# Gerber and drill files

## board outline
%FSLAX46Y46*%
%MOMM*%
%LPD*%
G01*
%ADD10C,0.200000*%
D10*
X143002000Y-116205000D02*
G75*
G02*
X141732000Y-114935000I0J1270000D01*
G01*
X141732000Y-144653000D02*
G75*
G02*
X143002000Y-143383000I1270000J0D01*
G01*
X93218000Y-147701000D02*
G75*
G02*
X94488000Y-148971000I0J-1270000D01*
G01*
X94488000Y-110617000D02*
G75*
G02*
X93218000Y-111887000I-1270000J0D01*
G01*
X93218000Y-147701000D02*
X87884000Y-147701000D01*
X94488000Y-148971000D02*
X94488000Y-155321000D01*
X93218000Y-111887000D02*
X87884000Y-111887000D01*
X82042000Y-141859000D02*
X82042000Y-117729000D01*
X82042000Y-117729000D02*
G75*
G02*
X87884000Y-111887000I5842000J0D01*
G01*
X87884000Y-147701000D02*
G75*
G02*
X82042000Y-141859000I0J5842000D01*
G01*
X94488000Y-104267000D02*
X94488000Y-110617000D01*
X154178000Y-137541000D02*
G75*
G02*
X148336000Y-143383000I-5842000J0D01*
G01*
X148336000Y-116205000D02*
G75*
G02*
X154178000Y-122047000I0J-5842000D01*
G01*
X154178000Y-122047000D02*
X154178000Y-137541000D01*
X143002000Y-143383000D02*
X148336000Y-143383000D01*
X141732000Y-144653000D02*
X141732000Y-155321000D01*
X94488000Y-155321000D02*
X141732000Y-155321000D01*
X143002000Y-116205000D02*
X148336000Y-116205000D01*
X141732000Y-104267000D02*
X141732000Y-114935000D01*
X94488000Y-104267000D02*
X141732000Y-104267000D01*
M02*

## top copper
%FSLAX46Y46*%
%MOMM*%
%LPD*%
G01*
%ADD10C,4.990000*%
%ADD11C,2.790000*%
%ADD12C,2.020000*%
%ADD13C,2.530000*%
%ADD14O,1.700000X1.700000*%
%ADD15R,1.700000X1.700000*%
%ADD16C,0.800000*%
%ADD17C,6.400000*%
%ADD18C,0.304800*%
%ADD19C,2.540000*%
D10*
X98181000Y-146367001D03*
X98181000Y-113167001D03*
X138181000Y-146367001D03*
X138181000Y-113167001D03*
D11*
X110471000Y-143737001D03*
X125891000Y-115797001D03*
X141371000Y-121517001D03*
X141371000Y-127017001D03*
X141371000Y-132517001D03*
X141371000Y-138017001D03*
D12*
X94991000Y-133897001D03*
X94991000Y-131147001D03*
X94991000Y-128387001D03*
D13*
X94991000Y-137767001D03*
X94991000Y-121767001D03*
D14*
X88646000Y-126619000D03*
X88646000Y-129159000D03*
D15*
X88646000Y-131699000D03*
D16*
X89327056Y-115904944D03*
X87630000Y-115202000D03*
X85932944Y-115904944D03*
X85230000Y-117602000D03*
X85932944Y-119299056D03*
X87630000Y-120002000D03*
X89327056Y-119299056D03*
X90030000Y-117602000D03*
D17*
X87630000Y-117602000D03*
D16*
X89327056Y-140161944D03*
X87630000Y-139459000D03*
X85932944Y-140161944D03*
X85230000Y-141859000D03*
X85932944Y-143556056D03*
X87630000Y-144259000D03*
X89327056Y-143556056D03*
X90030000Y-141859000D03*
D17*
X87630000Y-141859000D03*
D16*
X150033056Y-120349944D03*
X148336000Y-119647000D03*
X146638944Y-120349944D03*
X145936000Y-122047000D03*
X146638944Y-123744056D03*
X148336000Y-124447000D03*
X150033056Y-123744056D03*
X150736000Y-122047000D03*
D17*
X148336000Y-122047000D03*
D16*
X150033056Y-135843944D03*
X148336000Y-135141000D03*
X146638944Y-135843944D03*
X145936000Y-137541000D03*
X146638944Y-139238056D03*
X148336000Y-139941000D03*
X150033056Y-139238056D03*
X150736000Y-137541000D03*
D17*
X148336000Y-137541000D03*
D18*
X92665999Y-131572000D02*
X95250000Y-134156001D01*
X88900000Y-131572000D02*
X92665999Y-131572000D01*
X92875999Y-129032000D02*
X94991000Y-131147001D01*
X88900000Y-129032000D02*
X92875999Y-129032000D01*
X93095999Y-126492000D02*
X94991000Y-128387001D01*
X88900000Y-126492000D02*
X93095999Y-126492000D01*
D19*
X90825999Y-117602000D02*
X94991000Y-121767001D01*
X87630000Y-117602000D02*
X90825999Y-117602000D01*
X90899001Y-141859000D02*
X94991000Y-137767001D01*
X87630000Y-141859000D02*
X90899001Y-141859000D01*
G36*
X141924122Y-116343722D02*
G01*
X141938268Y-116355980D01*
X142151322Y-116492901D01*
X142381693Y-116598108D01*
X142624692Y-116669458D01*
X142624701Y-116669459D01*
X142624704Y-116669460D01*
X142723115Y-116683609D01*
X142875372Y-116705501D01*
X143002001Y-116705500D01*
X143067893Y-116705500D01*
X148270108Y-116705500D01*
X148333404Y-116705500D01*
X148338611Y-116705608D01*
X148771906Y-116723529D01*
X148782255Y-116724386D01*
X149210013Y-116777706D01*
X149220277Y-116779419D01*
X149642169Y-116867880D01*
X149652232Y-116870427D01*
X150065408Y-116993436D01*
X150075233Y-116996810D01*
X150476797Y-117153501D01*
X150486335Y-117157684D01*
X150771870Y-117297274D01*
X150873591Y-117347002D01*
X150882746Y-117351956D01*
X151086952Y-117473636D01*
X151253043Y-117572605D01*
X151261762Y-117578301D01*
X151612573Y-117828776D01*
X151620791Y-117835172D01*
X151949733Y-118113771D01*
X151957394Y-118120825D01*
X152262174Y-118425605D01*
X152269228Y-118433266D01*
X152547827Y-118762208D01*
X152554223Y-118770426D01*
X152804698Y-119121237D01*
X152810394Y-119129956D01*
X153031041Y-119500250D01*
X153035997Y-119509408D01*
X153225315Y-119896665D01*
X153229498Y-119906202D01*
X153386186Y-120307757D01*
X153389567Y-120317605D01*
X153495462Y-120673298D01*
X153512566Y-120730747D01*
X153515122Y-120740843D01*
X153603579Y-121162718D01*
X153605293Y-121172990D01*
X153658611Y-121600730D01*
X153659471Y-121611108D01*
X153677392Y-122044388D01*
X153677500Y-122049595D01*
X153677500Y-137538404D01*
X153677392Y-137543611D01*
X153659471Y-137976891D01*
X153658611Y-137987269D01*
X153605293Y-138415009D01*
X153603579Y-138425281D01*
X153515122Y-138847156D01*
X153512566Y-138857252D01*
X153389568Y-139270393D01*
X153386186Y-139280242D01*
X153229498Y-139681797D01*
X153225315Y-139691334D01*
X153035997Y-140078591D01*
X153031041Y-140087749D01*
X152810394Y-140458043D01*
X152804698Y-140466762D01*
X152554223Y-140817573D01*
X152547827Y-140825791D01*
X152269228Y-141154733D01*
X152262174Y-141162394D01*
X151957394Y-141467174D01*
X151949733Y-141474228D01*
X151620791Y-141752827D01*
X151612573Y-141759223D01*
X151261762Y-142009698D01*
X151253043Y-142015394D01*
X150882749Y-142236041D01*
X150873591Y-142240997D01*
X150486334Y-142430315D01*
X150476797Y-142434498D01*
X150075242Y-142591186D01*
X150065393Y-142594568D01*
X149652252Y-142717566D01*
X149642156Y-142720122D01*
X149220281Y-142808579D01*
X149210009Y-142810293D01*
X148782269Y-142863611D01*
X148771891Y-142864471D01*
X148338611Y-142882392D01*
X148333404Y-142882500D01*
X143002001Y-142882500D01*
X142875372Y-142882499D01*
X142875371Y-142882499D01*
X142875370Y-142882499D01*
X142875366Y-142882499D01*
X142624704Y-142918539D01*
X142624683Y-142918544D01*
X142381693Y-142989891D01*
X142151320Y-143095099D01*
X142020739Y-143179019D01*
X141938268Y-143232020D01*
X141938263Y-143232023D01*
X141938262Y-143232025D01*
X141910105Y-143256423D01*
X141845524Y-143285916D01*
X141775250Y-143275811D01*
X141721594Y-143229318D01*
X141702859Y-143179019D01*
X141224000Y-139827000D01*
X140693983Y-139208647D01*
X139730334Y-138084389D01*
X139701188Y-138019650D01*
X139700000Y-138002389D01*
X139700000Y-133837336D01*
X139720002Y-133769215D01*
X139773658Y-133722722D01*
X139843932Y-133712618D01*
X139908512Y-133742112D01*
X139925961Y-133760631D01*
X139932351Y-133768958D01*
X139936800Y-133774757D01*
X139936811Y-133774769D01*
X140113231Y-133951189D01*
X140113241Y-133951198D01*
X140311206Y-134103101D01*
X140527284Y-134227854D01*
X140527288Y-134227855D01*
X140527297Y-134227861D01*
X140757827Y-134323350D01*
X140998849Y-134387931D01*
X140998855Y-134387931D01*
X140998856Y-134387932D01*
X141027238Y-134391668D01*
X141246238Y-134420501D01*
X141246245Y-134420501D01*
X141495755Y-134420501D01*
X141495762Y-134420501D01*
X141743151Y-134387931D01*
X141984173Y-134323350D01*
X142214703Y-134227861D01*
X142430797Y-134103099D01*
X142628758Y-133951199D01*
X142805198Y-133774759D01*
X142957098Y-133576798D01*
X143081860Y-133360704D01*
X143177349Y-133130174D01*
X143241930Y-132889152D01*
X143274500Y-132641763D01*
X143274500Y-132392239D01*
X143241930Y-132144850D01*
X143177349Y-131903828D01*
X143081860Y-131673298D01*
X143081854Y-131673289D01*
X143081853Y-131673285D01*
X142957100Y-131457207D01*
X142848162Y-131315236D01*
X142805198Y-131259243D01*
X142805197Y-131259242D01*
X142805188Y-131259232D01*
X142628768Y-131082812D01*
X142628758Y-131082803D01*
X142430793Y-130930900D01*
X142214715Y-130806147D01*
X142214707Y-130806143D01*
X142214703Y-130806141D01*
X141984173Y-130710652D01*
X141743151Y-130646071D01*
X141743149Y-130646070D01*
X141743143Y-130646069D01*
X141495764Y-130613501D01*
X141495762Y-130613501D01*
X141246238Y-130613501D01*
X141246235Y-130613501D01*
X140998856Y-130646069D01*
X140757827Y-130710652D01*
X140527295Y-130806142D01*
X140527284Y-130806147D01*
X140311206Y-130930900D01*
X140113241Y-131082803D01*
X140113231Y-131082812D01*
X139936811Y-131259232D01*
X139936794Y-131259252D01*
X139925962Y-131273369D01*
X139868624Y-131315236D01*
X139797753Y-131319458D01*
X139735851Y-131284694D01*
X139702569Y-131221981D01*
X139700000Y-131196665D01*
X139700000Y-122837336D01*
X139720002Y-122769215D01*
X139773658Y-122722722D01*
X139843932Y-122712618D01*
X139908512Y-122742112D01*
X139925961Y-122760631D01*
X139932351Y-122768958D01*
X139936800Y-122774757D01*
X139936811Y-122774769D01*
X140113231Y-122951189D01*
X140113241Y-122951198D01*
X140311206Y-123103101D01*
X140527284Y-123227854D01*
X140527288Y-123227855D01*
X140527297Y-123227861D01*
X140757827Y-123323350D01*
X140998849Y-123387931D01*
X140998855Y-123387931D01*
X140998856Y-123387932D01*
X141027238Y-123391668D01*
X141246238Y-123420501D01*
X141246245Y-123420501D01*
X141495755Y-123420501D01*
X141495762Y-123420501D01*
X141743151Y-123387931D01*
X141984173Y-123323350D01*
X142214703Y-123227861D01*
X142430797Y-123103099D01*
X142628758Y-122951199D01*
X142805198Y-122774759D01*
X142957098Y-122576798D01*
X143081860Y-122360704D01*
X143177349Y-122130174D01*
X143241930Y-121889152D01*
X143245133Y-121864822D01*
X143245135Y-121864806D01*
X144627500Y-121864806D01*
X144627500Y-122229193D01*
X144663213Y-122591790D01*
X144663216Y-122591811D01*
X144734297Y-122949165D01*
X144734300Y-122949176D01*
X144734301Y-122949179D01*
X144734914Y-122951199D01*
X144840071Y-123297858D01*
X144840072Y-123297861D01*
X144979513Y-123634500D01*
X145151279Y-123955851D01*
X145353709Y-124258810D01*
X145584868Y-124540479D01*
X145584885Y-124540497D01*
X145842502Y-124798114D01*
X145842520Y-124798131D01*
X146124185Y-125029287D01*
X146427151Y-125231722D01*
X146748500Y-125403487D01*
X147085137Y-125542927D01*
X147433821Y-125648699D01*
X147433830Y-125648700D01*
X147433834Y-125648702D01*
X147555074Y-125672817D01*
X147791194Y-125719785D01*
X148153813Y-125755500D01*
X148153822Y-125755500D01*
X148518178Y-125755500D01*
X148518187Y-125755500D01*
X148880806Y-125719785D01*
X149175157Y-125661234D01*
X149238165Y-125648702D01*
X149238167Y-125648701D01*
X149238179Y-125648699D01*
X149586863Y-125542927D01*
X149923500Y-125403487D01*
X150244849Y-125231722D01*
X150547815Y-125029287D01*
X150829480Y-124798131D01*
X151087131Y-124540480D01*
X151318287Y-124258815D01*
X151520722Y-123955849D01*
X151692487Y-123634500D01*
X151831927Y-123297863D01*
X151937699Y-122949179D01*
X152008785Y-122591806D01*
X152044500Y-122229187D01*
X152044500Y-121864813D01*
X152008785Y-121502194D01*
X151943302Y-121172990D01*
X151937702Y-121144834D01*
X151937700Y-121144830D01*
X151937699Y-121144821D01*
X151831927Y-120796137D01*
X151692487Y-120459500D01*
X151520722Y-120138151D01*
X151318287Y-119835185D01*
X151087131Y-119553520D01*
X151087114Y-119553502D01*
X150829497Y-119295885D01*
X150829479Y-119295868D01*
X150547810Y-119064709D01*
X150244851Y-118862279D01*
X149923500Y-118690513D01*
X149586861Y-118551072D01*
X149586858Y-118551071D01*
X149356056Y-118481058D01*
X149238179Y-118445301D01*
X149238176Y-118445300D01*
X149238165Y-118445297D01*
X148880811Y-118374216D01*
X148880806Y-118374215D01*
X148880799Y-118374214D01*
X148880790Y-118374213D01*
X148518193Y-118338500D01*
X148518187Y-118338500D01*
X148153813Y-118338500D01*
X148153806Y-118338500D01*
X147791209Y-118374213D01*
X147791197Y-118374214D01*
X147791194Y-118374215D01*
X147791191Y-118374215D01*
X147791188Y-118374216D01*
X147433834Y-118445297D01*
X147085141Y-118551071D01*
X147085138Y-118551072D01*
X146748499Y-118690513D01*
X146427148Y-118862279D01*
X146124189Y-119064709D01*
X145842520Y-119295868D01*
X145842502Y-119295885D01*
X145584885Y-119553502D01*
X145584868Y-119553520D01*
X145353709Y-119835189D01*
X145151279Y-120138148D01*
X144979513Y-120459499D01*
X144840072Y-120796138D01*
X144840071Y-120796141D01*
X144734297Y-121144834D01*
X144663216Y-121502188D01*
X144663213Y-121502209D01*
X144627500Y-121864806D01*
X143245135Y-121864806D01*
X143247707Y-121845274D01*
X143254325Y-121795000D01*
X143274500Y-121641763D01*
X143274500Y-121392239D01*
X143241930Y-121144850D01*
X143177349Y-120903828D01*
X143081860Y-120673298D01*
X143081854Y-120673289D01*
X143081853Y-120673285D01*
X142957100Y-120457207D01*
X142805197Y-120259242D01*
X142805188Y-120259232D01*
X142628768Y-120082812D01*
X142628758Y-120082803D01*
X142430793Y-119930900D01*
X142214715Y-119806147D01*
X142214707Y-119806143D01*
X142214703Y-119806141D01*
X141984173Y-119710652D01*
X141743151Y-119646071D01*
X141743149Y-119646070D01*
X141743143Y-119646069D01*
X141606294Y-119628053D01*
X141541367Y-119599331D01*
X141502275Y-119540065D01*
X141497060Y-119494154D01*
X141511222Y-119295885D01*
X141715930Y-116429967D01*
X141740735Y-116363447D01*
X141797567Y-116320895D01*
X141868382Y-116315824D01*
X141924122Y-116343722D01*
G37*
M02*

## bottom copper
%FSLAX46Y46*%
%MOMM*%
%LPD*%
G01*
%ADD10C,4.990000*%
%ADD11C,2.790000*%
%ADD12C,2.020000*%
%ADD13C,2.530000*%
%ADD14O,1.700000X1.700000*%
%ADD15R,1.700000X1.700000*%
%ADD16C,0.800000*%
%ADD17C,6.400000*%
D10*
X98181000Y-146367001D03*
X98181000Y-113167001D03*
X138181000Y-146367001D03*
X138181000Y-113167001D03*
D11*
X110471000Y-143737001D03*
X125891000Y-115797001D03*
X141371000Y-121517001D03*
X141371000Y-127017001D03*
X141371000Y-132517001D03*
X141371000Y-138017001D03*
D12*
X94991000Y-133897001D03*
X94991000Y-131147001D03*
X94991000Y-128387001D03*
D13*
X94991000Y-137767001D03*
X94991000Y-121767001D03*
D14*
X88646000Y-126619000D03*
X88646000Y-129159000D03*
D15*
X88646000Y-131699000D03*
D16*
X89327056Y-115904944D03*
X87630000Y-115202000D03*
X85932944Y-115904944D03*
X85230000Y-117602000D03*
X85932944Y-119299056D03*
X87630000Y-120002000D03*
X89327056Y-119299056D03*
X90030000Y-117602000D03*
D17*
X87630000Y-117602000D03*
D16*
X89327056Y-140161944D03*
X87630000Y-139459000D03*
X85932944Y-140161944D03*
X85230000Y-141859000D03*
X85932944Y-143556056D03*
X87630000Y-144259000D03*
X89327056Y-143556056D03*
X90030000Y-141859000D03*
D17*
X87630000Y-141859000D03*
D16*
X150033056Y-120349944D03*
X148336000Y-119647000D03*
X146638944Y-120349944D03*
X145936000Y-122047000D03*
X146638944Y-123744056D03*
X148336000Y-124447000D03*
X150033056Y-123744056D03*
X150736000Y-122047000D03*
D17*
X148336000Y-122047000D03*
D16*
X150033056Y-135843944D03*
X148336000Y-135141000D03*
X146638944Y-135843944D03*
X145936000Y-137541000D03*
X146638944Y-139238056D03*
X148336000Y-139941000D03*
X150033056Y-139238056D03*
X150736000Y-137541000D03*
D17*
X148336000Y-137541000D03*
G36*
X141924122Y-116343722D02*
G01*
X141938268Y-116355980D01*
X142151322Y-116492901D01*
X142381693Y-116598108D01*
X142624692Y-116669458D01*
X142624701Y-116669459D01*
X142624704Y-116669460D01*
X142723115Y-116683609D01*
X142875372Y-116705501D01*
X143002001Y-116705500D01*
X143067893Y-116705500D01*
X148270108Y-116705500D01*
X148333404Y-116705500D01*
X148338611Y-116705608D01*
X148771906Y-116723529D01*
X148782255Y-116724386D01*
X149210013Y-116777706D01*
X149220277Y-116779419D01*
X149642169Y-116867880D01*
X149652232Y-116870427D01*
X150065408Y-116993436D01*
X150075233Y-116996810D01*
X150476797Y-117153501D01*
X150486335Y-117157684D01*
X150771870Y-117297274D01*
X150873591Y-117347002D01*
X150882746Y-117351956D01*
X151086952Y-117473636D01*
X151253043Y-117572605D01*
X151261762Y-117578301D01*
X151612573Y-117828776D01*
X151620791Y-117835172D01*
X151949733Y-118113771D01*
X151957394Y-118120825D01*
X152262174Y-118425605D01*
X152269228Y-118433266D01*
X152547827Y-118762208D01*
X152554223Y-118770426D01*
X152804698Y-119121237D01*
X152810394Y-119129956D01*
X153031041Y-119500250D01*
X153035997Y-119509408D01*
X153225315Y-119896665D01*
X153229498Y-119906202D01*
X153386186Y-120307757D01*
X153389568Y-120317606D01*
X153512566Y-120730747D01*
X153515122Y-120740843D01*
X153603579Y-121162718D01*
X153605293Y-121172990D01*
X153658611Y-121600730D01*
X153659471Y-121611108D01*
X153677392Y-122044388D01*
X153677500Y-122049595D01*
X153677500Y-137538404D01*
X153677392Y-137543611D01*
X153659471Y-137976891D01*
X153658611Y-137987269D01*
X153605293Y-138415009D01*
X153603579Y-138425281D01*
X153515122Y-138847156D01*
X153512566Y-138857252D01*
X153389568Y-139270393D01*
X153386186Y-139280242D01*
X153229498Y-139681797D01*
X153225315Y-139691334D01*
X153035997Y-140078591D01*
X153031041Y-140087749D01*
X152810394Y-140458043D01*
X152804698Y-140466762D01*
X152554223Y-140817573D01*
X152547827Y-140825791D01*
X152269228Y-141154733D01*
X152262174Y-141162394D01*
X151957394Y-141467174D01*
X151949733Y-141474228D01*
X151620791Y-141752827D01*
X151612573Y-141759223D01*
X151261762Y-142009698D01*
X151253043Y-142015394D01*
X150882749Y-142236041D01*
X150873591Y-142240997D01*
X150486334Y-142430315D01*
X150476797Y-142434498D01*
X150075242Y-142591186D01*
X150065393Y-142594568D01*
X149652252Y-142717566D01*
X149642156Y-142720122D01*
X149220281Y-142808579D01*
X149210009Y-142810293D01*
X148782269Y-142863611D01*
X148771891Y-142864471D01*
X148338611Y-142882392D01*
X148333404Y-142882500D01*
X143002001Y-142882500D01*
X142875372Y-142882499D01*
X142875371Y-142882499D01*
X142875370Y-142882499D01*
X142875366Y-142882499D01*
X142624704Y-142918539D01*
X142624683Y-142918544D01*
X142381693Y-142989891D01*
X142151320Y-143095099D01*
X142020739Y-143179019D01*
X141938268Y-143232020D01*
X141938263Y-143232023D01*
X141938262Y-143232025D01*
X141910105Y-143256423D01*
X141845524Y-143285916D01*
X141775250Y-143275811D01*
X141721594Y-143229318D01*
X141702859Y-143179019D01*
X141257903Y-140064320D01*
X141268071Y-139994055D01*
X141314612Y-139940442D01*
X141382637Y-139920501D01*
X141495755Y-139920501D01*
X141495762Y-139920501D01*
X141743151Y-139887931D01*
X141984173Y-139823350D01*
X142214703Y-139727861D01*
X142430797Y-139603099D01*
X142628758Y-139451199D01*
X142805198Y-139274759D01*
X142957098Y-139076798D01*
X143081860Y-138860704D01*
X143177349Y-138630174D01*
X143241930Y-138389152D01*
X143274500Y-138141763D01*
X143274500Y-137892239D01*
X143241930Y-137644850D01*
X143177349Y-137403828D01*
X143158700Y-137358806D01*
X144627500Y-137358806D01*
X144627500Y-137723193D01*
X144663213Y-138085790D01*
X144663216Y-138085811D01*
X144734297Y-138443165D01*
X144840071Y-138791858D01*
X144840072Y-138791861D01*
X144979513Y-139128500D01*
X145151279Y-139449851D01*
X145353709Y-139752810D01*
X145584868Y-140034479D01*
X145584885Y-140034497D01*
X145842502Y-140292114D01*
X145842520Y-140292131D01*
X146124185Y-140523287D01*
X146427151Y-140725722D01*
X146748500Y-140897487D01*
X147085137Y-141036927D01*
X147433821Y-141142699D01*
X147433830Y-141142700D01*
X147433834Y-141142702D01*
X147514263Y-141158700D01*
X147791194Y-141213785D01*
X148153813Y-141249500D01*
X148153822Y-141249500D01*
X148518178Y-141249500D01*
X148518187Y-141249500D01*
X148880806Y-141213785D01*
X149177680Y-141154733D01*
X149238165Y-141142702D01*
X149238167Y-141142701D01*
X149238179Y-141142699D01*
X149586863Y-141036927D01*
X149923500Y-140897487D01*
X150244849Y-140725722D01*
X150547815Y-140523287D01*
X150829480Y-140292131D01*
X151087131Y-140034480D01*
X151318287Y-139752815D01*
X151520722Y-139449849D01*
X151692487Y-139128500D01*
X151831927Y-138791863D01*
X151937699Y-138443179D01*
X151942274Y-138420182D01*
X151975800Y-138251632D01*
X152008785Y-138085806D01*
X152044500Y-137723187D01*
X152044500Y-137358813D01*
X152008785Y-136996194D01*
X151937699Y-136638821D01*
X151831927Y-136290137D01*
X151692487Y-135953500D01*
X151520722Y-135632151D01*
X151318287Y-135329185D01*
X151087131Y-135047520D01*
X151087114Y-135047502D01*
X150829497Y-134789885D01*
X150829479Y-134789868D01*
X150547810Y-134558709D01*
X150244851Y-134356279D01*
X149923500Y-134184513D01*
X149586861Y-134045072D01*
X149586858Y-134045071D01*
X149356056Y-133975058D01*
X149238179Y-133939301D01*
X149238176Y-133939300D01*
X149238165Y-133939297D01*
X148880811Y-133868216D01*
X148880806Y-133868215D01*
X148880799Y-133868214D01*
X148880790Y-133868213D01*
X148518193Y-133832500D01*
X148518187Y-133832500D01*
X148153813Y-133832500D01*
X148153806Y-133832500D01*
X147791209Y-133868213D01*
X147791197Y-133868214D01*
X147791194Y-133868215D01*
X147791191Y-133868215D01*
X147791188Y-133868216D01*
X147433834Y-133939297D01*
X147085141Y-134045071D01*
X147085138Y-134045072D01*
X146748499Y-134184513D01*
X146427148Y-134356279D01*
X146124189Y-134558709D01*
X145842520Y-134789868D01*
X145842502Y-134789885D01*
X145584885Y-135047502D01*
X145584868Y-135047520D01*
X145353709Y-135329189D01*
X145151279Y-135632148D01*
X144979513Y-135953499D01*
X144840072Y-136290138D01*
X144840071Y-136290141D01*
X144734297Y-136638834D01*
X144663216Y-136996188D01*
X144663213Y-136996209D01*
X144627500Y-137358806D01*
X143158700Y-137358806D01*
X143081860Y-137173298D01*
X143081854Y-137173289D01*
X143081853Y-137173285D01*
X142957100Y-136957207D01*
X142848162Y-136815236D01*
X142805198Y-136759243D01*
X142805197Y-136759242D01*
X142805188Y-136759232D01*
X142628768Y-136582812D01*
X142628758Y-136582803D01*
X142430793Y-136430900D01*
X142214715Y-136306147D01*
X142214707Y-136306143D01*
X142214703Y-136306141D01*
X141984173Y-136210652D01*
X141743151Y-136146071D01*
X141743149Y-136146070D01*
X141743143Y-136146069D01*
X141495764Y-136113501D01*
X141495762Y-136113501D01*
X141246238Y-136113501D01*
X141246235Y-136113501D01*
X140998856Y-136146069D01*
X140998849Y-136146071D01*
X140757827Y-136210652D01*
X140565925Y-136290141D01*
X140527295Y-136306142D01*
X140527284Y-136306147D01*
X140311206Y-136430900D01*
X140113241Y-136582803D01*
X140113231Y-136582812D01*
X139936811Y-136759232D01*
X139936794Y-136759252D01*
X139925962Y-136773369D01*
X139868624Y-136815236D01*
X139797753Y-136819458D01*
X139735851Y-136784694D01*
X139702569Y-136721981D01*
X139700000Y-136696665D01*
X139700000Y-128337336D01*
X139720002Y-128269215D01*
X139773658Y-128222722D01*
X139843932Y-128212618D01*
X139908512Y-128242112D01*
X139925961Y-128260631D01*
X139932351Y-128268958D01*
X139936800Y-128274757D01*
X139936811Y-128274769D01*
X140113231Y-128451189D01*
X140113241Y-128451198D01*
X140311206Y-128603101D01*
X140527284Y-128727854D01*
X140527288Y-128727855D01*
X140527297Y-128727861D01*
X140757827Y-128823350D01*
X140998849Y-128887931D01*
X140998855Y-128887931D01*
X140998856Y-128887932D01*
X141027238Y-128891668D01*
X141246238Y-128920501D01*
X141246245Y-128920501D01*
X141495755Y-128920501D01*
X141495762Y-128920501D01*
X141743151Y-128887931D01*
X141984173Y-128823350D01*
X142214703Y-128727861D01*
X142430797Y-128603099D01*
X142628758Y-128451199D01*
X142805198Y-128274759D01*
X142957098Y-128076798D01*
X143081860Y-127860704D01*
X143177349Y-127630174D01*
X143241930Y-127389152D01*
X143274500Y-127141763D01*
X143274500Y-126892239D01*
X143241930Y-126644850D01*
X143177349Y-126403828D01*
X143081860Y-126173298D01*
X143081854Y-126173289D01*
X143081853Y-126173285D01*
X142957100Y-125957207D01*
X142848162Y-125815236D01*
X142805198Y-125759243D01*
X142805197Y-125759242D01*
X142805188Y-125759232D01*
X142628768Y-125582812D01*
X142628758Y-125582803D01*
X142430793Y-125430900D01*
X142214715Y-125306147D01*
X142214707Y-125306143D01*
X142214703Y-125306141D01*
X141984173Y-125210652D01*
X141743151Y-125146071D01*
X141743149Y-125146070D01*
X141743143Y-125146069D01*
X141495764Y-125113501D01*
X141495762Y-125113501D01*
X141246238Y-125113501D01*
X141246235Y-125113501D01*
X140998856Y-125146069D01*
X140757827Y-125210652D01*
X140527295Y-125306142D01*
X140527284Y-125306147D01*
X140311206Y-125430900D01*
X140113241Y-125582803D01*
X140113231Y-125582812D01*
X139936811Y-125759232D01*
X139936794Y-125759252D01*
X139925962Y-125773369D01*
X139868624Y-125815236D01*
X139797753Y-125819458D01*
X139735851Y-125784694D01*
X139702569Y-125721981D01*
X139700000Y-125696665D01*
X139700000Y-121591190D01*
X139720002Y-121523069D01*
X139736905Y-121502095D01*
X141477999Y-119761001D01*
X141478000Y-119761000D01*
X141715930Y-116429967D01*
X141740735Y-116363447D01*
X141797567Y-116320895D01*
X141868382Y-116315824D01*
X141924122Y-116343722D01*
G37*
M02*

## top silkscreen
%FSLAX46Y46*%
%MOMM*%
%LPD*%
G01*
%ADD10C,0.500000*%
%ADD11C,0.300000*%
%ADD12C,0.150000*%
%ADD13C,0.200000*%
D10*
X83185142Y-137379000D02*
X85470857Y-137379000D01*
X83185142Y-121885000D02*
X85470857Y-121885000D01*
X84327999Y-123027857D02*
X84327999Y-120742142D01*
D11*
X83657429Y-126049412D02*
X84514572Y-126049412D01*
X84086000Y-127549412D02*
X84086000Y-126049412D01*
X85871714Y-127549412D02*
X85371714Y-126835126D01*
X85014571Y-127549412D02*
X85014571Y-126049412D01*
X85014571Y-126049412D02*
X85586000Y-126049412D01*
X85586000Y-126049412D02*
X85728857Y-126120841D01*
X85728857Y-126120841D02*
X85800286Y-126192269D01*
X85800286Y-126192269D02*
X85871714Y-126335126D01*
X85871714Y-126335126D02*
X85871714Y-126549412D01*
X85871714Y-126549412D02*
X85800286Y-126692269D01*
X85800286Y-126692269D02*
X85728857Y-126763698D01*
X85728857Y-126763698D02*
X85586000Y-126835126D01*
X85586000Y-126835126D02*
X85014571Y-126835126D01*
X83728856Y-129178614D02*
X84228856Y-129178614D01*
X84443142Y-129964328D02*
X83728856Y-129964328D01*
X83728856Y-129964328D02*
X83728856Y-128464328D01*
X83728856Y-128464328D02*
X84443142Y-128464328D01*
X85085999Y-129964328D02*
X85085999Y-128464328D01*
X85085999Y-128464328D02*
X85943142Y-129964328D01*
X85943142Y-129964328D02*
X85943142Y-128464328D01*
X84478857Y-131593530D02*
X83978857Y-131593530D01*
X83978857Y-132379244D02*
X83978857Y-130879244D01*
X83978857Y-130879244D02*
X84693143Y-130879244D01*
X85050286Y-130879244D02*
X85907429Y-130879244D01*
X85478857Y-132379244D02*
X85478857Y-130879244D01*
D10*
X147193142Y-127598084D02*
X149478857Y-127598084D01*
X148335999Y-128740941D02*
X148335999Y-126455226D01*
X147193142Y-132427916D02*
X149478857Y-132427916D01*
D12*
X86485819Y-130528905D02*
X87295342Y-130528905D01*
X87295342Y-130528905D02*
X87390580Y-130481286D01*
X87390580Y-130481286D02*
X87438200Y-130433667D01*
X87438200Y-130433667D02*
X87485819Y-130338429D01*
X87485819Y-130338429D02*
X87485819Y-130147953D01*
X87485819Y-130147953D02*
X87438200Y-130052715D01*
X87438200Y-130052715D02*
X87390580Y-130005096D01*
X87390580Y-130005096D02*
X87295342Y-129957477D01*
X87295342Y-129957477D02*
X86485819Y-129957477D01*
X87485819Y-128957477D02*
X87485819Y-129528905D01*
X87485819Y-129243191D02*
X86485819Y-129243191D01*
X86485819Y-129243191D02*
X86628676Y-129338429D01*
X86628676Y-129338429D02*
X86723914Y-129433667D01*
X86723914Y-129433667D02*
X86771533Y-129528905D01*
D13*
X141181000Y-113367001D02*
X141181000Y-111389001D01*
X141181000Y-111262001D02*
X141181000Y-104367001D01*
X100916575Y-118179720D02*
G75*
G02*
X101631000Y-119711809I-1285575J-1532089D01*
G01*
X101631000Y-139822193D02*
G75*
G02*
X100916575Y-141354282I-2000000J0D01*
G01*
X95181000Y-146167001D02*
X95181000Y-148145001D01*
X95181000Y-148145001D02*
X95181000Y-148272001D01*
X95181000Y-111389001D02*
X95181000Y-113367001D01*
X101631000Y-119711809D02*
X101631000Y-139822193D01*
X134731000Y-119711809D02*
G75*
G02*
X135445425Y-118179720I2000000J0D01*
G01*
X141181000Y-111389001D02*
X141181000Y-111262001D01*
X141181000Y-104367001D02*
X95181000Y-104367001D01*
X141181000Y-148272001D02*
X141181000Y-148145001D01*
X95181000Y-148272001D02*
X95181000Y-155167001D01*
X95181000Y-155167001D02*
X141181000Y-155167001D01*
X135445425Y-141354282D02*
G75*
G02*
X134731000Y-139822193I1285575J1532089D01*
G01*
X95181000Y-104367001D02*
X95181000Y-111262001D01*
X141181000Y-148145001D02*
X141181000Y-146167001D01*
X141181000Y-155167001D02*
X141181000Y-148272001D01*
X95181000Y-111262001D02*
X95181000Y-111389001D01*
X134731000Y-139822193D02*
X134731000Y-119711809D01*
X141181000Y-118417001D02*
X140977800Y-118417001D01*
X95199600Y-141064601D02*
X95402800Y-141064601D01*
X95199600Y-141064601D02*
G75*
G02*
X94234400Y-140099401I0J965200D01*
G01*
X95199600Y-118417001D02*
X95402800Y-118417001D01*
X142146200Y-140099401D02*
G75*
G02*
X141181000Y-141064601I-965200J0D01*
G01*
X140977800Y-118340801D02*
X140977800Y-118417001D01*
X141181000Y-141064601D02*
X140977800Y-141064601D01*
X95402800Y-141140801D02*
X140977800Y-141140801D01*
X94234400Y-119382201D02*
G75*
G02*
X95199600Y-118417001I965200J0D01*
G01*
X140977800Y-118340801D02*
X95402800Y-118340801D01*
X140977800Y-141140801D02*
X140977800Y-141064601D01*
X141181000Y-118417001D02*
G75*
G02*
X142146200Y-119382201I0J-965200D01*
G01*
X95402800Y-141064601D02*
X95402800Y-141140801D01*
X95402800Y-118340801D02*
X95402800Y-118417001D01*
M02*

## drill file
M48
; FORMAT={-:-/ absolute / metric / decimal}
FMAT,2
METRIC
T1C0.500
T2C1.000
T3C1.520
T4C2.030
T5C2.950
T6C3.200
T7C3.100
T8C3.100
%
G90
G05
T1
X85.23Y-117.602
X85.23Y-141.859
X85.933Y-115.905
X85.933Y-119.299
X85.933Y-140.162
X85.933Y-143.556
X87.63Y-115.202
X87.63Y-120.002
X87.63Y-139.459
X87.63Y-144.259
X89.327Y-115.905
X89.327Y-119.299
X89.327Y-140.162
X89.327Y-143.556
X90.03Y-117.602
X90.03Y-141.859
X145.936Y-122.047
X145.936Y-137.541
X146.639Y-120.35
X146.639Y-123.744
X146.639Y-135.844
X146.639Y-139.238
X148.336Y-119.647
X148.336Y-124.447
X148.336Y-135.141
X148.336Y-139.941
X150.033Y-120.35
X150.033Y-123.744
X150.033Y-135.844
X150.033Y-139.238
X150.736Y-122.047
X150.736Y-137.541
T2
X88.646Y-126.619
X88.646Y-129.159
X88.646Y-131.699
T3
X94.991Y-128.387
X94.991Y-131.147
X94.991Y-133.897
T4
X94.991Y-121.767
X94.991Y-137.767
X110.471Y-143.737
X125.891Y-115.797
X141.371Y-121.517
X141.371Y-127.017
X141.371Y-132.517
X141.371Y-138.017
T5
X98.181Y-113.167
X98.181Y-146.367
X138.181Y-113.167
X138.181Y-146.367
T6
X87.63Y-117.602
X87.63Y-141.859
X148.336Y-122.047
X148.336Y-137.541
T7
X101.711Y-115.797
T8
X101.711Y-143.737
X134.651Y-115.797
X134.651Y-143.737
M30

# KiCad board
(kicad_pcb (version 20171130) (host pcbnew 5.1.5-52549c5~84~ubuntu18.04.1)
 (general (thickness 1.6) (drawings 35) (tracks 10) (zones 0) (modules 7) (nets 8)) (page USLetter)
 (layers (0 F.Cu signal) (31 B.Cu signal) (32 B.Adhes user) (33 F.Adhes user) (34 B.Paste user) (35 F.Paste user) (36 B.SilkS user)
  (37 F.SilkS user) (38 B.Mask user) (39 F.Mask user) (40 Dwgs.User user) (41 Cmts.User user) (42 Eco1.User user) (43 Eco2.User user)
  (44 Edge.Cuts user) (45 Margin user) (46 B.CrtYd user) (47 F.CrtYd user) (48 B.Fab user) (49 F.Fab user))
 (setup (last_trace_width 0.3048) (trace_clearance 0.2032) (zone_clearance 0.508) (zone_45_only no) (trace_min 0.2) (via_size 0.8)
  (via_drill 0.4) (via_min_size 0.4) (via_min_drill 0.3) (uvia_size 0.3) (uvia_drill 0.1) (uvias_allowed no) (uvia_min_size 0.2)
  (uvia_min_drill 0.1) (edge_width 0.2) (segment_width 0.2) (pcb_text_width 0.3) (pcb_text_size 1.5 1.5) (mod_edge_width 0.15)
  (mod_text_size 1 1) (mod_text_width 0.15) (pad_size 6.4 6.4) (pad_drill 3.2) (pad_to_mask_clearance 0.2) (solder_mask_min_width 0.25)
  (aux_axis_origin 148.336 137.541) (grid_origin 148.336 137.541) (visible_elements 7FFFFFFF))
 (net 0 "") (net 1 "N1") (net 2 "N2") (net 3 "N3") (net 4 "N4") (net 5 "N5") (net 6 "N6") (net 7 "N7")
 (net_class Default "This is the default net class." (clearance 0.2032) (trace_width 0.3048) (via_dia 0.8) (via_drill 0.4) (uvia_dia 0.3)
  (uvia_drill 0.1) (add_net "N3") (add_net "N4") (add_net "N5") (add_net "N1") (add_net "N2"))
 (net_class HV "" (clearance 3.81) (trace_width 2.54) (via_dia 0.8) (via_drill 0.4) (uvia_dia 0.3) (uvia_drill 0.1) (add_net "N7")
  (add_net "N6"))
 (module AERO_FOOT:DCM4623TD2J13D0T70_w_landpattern (layer F.Cu) (at 118.181 129.767001)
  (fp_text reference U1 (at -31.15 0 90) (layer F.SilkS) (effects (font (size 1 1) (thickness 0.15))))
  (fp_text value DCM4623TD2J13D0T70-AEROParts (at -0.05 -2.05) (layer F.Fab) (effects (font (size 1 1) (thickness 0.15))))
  (fp_line (start 23 -16.4) (end 23 -18.378) (layer F.SilkS) (width 0.2))
  (fp_line (start 23 -18.505) (end 23 -25.4) (layer F.SilkS) (width 0.2))
  (fp_arc (start -18.55 -10.055192) (end -16.55 -10.055192) (angle -50) (layer F.SilkS) (width 0.2))
  (fp_arc (start -18.55 10.055192) (end -17.264425 11.587281) (angle -50) (layer F.SilkS) (width 0.2))
  (fp_line (start -23 16.4) (end -23 18.378) (layer F.SilkS) (width 0.2))
  (fp_line (start -23 18.378) (end -23 18.505) (layer F.SilkS) (width 0.2))
  (fp_line (start -23 -18.378) (end -23 -16.4) (layer F.SilkS) (width 0.2))
  (fp_line (start -16.55 -10.055192) (end -16.55 10.055192) (layer F.SilkS) (width 0.2))
  (fp_arc (start 18.55 -10.055192) (end 17.264425 -11.587281) (angle -50) (layer F.SilkS) (width 0.2))
  (fp_line (start 23 -18.378) (end 23 -18.505) (layer F.SilkS) (width 0.2))
  (fp_line (start 23 -25.4) (end -23 -25.4) (layer F.SilkS) (width 0.2))
  (fp_line (start 23 18.505) (end 23 18.378) (layer F.SilkS) (width 0.2))
  (fp_line (start -23 18.505) (end -23 25.4) (layer F.SilkS) (width 0.2))
  (fp_line (start -23 25.4) (end 23 25.4) (layer F.SilkS) (width 0.2))
  (fp_arc (start 18.55 10.055192) (end 16.55 10.055192) (angle -50) (layer F.SilkS) (width 0.2))
  (fp_line (start -23 -25.4) (end -23 -18.505) (layer F.SilkS) (width 0.2))
  (fp_line (start 23 18.378) (end 23 16.4) (layer F.SilkS) (width 0.2))
  (fp_line (start 23 25.4) (end 23 18.505) (layer F.SilkS) (width 0.2))
  (fp_line (start -23 -18.505) (end -23 -18.378) (layer F.SilkS) (width 0.2))
  (fp_line (start 16.55 10.055192) (end 16.55 -10.055192) (layer F.SilkS) (width 0.2))
  (fp_line (start 23 -11.35) (end 22.7968 -11.35) (layer F.SilkS) (width 0.2))
  (fp_line (start -22.9814 11.2976) (end -22.7782 11.2976) (layer F.SilkS) (width 0.2))
  (fp_arc (start -22.9814 10.3324) (end -23.9466 10.3324) (angle -90) (layer F.SilkS) (width 0.2))
  (fp_line (start -22.9814 -11.35) (end -22.7782 -11.35) (layer F.SilkS) (width 0.2))
  (fp_arc (start 23 10.3324) (end 23 11.2976) (angle -90) (layer F.SilkS) (width 0.2))
  (fp_line (start 22.7968 -11.4262) (end 22.7968 -11.35) (layer F.SilkS) (width 0.2))
  (fp_line (start 23 11.2976) (end 22.7968 11.2976) (layer F.SilkS) (width 0.2))
  (fp_line (start -22.7782 11.3738) (end 22.7968 11.3738) (layer F.SilkS) (width 0.2))
  (fp_arc (start -22.9814 -10.3848) (end -22.9814 -11.35) (angle -90) (layer F.SilkS) (width 0.2))
  (fp_line (start 22.7968 -11.4262) (end -22.7782 -11.4262) (layer F.SilkS) (width 0.2))
  (fp_line (start 22.7968 11.3738) (end 22.7968 11.2976) (layer F.SilkS) (width 0.2))
  (fp_arc (start 23 -10.3848) (end 23.9652 -10.3848) (angle -90) (layer F.SilkS) (width 0.2))
  (fp_line (start -22.7782 11.2976) (end -22.7782 11.3738) (layer F.SilkS) (width 0.2))
  (fp_line (start -22.7782 -11.4262) (end -22.7782 -11.35) (layer F.SilkS) (width 0.2))
  (pad 14 thru_hole circle (at -20 16.6) (size 4.99 4.99) (drill 2.949999) (layers *.Cu *.Mask))
  (pad 12 thru_hole circle (at -20 -16.6) (size 4.99 4.99) (drill 2.949999) (layers *.Cu *.Mask))
  (pad 15 thru_hole circle (at 20 16.6) (size 4.99 4.99) (drill 2.949999) (layers *.Cu *.Mask))
  (pad 13 thru_hole circle (at 20 -16.6) (size 4.99 4.99) (drill 2.949999) (layers *.Cu *.Mask))
  (pad 10 thru_hole circle (at -7.71 13.97) (size 2.79 2.79) (drill 2.03) (layers *.Cu *.Mask))
  (pad 11 thru_hole circle (at 7.71 -13.97) (size 2.79 2.79) (drill 2.03) (layers *.Cu *.Mask))
  (pad "" np_thru_hole circle (at 16.47 13.97) (size 3.1 3.1) (drill 3.1) (layers *.Cu *.Mask))
  (pad "" np_thru_hole circle (at -16.47 13.97) (size 3.1 3.1) (drill 3.1) (layers *.Cu *.Mask))
  (pad "" np_thru_hole circle (at -16.47 -13.97) (size 3.099999 3.099999) (drill 3.099999) (layers *.Cu *.Mask))
  (pad "" np_thru_hole circle (at 16.47 -13.97) (size 3.1 3.1) (drill 3.1) (layers *.Cu *.Mask))
  (pad 9 thru_hole circle (at 23.19 -8.25) (size 2.79 2.79) (drill 2.03) (layers *.Cu *.Mask) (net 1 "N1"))
  (pad 8 thru_hole circle (at 23.19 -2.75) (size 2.79 2.79) (drill 2.03) (layers *.Cu *.Mask) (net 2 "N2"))
  (pad 7 thru_hole circle (at 23.19 2.75) (size 2.79 2.79) (drill 2.03) (layers *.Cu *.Mask) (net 1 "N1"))
  (pad 6 thru_hole circle (at 23.19 8.25) (size 2.79 2.79) (drill 2.03) (layers *.Cu *.Mask) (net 2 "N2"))
  (pad 4 thru_hole circle (at -23.19 4.13) (size 2.02 2.02) (drill 1.52) (layers *.Cu *.Mask) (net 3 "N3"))
  (pad 3 thru_hole circle (at -23.19 1.38) (size 2.02 2.02) (drill 1.52) (layers *.Cu *.Mask) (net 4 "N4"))
  (pad 2 thru_hole circle (at -23.19 -1.38) (size 2.02 2.02) (drill 1.52) (layers *.Cu *.Mask) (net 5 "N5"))
  (pad 5 thru_hole circle (at -23.19 8) (size 2.53 2.53) (drill 2.03) (layers *.Cu *.Mask) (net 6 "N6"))
  (pad 1 thru_hole circle (at -23.19 -8) (size 2.53 2.53) (drill 2.03) (layers *.Cu *.Mask) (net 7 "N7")))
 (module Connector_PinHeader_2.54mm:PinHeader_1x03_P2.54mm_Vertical (layer B.Cu) (at 88.646 131.699)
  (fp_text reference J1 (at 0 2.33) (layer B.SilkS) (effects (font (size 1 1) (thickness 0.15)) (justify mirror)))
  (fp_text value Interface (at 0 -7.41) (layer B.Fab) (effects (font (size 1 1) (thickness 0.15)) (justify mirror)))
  (pad 3 thru_hole oval (at 0 -5.08) (size 1.7 1.7) (drill 1) (layers *.Cu *.Mask) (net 5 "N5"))
  (pad 2 thru_hole oval (at 0 -2.54) (size 1.7 1.7) (drill 1) (layers *.Cu *.Mask) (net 4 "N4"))
  (pad 1 thru_hole rect (at 0 0) (size 1.7 1.7) (drill 1) (layers *.Cu *.Mask) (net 3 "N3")))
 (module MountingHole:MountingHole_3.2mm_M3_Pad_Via (layer F.Cu) (at 87.63 117.602)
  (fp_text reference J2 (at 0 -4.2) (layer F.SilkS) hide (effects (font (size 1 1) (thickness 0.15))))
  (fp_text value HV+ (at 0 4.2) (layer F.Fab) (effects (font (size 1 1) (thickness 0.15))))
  (pad 1 thru_hole circle (at 1.697056 -1.697056) (size 0.8 0.8) (drill 0.5) (layers *.Cu *.Mask) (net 7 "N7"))
  (pad 1 thru_hole circle (at 0 -2.4) (size 0.8 0.8) (drill 0.5) (layers *.Cu *.Mask) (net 7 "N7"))
  (pad 1 thru_hole circle (at -1.697056 -1.697056) (size 0.8 0.8) (drill 0.5) (layers *.Cu *.Mask) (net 7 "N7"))
  (pad 1 thru_hole circle (at -2.4 0) (size 0.8 0.8) (drill 0.5) (layers *.Cu *.Mask) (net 7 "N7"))
  (pad 1 thru_hole circle (at -1.697056 1.697056) (size 0.8 0.8) (drill 0.5) (layers *.Cu *.Mask) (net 7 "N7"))
  (pad 1 thru_hole circle (at 0 2.4) (size 0.8 0.8) (drill 0.5) (layers *.Cu *.Mask) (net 7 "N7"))
  (pad 1 thru_hole circle (at 1.697056 1.697056) (size 0.8 0.8) (drill 0.5) (layers *.Cu *.Mask) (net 7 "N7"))
  (pad 1 thru_hole circle (at 2.4 0) (size 0.8 0.8) (drill 0.5) (layers *.Cu *.Mask) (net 7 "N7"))
  (pad 1 thru_hole circle (at 0 0) (size 6.4 6.4) (drill 3.2) (layers *.Cu *.Mask) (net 7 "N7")))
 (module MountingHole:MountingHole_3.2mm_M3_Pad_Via (layer F.Cu) (at 87.63 141.859)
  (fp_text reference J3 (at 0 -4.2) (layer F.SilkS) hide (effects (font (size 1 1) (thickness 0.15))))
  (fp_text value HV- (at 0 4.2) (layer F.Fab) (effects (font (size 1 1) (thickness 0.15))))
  (pad 1 thru_hole circle (at 1.697056 -1.697056) (size 0.8 0.8) (drill 0.5) (layers *.Cu *.Mask) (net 6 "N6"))
  (pad 1 thru_hole circle (at 0 -2.4) (size 0.8 0.8) (drill 0.5) (layers *.Cu *.Mask) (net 6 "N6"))
  (pad 1 thru_hole circle (at -1.697056 -1.697056) (size 0.8 0.8) (drill 0.5) (layers *.Cu *.Mask) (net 6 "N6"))
  (pad 1 thru_hole circle (at -2.4 0) (size 0.8 0.8) (drill 0.5) (layers *.Cu *.Mask) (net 6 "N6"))
  (pad 1 thru_hole circle (at -1.697056 1.697056) (size 0.8 0.8) (drill 0.5) (layers *.Cu *.Mask) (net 6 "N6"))
  (pad 1 thru_hole circle (at 0 2.4) (size 0.8 0.8) (drill 0.5) (layers *.Cu *.Mask) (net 6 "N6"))
  (pad 1 thru_hole circle (at 1.697056 1.697056) (size 0.8 0.8) (drill 0.5) (layers *.Cu *.Mask) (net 6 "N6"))
  (pad 1 thru_hole circle (at 2.4 0) (size 0.8 0.8) (drill 0.5) (layers *.Cu *.Mask) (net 6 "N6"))
  (pad 1 thru_hole circle (at 0 0) (size 6.4 6.4) (drill 3.2) (layers *.Cu *.Mask) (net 6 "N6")))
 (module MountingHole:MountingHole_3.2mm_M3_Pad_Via (layer F.Cu) (at 148.336 122.047)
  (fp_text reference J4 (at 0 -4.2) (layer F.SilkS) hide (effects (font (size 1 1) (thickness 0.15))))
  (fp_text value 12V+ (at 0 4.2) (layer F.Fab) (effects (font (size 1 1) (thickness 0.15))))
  (pad 1 thru_hole circle (at 1.697056 -1.697056) (size 0.8 0.8) (drill 0.5) (layers *.Cu *.Mask) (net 1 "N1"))
  (pad 1 thru_hole circle (at 0 -2.4) (size 0.8 0.8) (drill 0.5) (layers *.Cu *.Mask) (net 1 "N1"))
  (pad 1 thru_hole circle (at -1.697056 -1.697056) (size 0.8 0.8) (drill 0.5) (layers *.Cu *.Mask) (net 1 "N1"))
  (pad 1 thru_hole circle (at -2.4 0) (size 0.8 0.8) (drill 0.5) (layers *.Cu *.Mask) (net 1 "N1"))
  (pad 1 thru_hole circle (at -1.697056 1.697056) (size 0.8 0.8) (drill 0.5) (layers *.Cu *.Mask) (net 1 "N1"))
  (pad 1 thru_hole circle (at 0 2.4) (size 0.8 0.8) (drill 0.5) (layers *.Cu *.Mask) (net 1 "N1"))
  (pad 1 thru_hole circle (at 1.697056 1.697056) (size 0.8 0.8) (drill 0.5) (layers *.Cu *.Mask) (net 1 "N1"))
  (pad 1 thru_hole circle (at 2.4 0) (size 0.8 0.8) (drill 0.5) (layers *.Cu *.Mask) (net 1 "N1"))
  (pad 1 thru_hole circle (at 0 0) (size 6.4 6.4) (drill 3.2) (layers *.Cu *.Mask) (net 1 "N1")))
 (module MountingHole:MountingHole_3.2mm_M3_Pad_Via (layer F.Cu) (at 148.336 137.541)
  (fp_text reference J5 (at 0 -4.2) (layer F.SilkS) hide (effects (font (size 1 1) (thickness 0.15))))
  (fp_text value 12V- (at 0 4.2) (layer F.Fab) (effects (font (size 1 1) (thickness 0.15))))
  (pad 1 thru_hole circle (at 1.697056 -1.697056) (size 0.8 0.8) (drill 0.5) (layers *.Cu *.Mask) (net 2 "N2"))
  (pad 1 thru_hole circle (at 0 -2.4) (size 0.8 0.8) (drill 0.5) (layers *.Cu *.Mask) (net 2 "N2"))
  (pad 1 thru_hole circle (at -1.697056 -1.697056) (size 0.8 0.8) (drill 0.5) (layers *.Cu *.Mask) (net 2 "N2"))
  (pad 1 thru_hole circle (at -2.4 0) (size 0.8 0.8) (drill 0.5) (layers *.Cu *.Mask) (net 2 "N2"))
  (pad 1 thru_hole circle (at -1.697056 1.697056) (size 0.8 0.8) (drill 0.5) (layers *.Cu *.Mask) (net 2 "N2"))
  (pad 1 thru_hole circle (at 0 2.4) (size 0.8 0.8) (drill 0.5) (layers *.Cu *.Mask) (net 2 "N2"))
  (pad 1 thru_hole circle (at 1.697056 1.697056) (size 0.8 0.8) (drill 0.5) (layers *.Cu *.Mask) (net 2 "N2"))
  (pad 1 thru_hole circle (at 2.4 0) (size 0.8 0.8) (drill 0.5) (layers *.Cu *.Mask) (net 2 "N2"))
  (pad 1 thru_hole circle (at 0 0) (size 6.4 6.4) (drill 3.2) (layers *.Cu *.Mask) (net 2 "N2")))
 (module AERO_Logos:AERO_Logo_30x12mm (layer B.Cu) (at 118.618 129.032 180)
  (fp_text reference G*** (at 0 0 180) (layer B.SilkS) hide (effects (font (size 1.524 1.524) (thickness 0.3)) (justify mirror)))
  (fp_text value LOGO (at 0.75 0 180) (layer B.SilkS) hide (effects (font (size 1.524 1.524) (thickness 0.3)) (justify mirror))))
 (gr_arc (start 143.002 114.935) (end 141.732 114.935) (angle -90) (layer Edge.Cuts) (width 0.2))
 (gr_arc (start 143.002 144.653) (end 143.002 143.383) (angle -90) (layer Edge.Cuts) (width 0.2))
 (gr_arc (start 93.218 148.971) (end 94.488 148.971) (angle -90) (layer Edge.Cuts) (width 0.2))
 (gr_arc (start 93.218 110.617) (end 93.218 111.887) (angle -90) (layer Edge.Cuts) (width 0.2))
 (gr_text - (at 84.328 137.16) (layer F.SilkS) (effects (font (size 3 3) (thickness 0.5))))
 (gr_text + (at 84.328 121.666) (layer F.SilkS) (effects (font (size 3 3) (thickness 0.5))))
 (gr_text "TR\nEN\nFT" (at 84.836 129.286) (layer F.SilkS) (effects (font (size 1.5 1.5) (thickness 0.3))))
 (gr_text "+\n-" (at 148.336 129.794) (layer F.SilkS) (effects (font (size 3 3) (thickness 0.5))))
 (gr_line (start 93.218 147.701) (end 87.884 147.701) (layer Edge.Cuts) (width 0.2))
 (gr_line (start 94.488 148.971) (end 94.488 155.321) (layer Edge.Cuts) (width 0.2))
 (gr_line (start 93.218 111.887) (end 87.884 111.887) (layer Edge.Cuts) (width 0.2))
 (gr_line (start 82.042 141.859) (end 82.042 117.729) (layer Edge.Cuts) (width 0.2))
 (gr_arc (start 87.884 117.729) (end 87.884 111.887) (angle -90) (layer Edge.Cuts) (width 0.2))
 (gr_arc (start 87.884 141.859) (end 82.042 141.859) (angle -90) (layer Edge.Cuts) (width 0.2))
 (gr_line (start 94.488 104.267) (end 94.488 110.617) (layer Edge.Cuts) (width 0.2))
 (gr_arc (start 148.336 137.541) (end 148.336 143.383) (angle -90) (layer Edge.Cuts) (width 0.2))
 (gr_arc (start 148.336 122.047) (end 154.178 122.047) (angle -90) (layer Edge.Cuts) (width 0.2))
 (gr_line (start 154.178 122.047) (end 154.178 137.541) (layer Edge.Cuts) (width 0.2))
 (gr_line (start 143.002 143.383) (end 148.336 143.383) (layer Edge.Cuts) (width 0.2))
 (gr_line (start 141.732 144.653) (end 141.732 155.321) (layer Edge.Cuts) (width 0.2))
 (gr_line (start 94.488 155.321) (end 141.732 155.321) (layer Edge.Cuts) (width 0.2))
 (gr_line (start 143.002 116.205) (end 148.336 116.205) (layer Edge.Cuts) (width 0.2))
 (gr_line (start 141.732 104.267) (end 141.732 114.935) (layer Edge.Cuts) (width 0.2))
 (gr_line (start 94.488 104.267) (end 141.732 104.267) (layer Edge.Cuts) (width 0.2))
 (segment (start 92.665999 131.572) (end 95.25 134.156001) (width 0.3048) (layer F.Cu) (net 3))
 (segment (start 88.9 131.572) (end 92.665999 131.572) (width 0.3048) (layer F.Cu) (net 3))
 (segment (start 92.875999 129.032) (end 94.991 131.147001) (width 0.3048) (layer F.Cu) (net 4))
 (segment (start 88.9 129.032) (end 92.875999 129.032) (width 0.3048) (layer F.Cu) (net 4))
 (segment (start 93.095999 126.492) (end 94.991 128.387001) (width 0.3048) (layer F.Cu) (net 5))
 (segment (start 88.9 126.492) (end 93.095999 126.492) (width 0.3048) (layer F.Cu) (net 5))
 (segment (start 90.825999 117.602) (end 94.991 121.767001) (width 2.54) (layer F.Cu) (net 7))
 (segment (start 87.63 117.602) (end 90.825999 117.602) (width 2.54) (layer F.Cu) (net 7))
 (segment (start 90.899001 141.859) (end 94.991 137.767001) (width 2.54) (layer F.Cu) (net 6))
 (segment (start 87.63 141.859) (end 90.899001 141.859) (width 2.54) (layer F.Cu) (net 6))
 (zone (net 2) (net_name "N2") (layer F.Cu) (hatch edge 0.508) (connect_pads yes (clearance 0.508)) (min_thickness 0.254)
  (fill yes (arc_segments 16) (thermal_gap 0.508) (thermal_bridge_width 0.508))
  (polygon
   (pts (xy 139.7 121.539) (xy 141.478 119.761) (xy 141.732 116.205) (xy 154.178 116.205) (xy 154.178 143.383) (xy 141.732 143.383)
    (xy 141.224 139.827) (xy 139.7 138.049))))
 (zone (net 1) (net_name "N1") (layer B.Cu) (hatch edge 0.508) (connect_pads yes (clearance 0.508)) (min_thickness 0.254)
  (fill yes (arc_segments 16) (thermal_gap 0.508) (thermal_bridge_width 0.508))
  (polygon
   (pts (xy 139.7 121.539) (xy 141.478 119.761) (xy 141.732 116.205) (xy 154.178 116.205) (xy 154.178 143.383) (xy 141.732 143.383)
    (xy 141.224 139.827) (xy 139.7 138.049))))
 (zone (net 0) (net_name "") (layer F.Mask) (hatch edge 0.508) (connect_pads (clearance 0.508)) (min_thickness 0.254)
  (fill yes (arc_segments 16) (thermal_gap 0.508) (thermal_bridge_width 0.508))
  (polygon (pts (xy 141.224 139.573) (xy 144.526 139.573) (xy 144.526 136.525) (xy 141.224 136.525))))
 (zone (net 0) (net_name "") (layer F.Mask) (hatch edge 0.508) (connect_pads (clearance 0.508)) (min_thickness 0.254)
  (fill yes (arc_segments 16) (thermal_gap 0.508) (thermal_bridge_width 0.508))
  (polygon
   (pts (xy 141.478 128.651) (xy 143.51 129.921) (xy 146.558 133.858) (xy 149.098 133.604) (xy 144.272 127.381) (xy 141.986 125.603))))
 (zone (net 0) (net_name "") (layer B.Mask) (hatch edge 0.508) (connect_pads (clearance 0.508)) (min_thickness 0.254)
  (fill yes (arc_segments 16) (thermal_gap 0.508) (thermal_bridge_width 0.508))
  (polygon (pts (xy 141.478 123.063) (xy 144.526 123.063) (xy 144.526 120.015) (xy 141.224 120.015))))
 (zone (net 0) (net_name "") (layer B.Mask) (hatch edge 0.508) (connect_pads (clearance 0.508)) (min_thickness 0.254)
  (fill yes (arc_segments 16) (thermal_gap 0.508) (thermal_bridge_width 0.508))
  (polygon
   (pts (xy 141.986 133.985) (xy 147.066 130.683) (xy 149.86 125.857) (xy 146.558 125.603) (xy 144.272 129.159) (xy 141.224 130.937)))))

